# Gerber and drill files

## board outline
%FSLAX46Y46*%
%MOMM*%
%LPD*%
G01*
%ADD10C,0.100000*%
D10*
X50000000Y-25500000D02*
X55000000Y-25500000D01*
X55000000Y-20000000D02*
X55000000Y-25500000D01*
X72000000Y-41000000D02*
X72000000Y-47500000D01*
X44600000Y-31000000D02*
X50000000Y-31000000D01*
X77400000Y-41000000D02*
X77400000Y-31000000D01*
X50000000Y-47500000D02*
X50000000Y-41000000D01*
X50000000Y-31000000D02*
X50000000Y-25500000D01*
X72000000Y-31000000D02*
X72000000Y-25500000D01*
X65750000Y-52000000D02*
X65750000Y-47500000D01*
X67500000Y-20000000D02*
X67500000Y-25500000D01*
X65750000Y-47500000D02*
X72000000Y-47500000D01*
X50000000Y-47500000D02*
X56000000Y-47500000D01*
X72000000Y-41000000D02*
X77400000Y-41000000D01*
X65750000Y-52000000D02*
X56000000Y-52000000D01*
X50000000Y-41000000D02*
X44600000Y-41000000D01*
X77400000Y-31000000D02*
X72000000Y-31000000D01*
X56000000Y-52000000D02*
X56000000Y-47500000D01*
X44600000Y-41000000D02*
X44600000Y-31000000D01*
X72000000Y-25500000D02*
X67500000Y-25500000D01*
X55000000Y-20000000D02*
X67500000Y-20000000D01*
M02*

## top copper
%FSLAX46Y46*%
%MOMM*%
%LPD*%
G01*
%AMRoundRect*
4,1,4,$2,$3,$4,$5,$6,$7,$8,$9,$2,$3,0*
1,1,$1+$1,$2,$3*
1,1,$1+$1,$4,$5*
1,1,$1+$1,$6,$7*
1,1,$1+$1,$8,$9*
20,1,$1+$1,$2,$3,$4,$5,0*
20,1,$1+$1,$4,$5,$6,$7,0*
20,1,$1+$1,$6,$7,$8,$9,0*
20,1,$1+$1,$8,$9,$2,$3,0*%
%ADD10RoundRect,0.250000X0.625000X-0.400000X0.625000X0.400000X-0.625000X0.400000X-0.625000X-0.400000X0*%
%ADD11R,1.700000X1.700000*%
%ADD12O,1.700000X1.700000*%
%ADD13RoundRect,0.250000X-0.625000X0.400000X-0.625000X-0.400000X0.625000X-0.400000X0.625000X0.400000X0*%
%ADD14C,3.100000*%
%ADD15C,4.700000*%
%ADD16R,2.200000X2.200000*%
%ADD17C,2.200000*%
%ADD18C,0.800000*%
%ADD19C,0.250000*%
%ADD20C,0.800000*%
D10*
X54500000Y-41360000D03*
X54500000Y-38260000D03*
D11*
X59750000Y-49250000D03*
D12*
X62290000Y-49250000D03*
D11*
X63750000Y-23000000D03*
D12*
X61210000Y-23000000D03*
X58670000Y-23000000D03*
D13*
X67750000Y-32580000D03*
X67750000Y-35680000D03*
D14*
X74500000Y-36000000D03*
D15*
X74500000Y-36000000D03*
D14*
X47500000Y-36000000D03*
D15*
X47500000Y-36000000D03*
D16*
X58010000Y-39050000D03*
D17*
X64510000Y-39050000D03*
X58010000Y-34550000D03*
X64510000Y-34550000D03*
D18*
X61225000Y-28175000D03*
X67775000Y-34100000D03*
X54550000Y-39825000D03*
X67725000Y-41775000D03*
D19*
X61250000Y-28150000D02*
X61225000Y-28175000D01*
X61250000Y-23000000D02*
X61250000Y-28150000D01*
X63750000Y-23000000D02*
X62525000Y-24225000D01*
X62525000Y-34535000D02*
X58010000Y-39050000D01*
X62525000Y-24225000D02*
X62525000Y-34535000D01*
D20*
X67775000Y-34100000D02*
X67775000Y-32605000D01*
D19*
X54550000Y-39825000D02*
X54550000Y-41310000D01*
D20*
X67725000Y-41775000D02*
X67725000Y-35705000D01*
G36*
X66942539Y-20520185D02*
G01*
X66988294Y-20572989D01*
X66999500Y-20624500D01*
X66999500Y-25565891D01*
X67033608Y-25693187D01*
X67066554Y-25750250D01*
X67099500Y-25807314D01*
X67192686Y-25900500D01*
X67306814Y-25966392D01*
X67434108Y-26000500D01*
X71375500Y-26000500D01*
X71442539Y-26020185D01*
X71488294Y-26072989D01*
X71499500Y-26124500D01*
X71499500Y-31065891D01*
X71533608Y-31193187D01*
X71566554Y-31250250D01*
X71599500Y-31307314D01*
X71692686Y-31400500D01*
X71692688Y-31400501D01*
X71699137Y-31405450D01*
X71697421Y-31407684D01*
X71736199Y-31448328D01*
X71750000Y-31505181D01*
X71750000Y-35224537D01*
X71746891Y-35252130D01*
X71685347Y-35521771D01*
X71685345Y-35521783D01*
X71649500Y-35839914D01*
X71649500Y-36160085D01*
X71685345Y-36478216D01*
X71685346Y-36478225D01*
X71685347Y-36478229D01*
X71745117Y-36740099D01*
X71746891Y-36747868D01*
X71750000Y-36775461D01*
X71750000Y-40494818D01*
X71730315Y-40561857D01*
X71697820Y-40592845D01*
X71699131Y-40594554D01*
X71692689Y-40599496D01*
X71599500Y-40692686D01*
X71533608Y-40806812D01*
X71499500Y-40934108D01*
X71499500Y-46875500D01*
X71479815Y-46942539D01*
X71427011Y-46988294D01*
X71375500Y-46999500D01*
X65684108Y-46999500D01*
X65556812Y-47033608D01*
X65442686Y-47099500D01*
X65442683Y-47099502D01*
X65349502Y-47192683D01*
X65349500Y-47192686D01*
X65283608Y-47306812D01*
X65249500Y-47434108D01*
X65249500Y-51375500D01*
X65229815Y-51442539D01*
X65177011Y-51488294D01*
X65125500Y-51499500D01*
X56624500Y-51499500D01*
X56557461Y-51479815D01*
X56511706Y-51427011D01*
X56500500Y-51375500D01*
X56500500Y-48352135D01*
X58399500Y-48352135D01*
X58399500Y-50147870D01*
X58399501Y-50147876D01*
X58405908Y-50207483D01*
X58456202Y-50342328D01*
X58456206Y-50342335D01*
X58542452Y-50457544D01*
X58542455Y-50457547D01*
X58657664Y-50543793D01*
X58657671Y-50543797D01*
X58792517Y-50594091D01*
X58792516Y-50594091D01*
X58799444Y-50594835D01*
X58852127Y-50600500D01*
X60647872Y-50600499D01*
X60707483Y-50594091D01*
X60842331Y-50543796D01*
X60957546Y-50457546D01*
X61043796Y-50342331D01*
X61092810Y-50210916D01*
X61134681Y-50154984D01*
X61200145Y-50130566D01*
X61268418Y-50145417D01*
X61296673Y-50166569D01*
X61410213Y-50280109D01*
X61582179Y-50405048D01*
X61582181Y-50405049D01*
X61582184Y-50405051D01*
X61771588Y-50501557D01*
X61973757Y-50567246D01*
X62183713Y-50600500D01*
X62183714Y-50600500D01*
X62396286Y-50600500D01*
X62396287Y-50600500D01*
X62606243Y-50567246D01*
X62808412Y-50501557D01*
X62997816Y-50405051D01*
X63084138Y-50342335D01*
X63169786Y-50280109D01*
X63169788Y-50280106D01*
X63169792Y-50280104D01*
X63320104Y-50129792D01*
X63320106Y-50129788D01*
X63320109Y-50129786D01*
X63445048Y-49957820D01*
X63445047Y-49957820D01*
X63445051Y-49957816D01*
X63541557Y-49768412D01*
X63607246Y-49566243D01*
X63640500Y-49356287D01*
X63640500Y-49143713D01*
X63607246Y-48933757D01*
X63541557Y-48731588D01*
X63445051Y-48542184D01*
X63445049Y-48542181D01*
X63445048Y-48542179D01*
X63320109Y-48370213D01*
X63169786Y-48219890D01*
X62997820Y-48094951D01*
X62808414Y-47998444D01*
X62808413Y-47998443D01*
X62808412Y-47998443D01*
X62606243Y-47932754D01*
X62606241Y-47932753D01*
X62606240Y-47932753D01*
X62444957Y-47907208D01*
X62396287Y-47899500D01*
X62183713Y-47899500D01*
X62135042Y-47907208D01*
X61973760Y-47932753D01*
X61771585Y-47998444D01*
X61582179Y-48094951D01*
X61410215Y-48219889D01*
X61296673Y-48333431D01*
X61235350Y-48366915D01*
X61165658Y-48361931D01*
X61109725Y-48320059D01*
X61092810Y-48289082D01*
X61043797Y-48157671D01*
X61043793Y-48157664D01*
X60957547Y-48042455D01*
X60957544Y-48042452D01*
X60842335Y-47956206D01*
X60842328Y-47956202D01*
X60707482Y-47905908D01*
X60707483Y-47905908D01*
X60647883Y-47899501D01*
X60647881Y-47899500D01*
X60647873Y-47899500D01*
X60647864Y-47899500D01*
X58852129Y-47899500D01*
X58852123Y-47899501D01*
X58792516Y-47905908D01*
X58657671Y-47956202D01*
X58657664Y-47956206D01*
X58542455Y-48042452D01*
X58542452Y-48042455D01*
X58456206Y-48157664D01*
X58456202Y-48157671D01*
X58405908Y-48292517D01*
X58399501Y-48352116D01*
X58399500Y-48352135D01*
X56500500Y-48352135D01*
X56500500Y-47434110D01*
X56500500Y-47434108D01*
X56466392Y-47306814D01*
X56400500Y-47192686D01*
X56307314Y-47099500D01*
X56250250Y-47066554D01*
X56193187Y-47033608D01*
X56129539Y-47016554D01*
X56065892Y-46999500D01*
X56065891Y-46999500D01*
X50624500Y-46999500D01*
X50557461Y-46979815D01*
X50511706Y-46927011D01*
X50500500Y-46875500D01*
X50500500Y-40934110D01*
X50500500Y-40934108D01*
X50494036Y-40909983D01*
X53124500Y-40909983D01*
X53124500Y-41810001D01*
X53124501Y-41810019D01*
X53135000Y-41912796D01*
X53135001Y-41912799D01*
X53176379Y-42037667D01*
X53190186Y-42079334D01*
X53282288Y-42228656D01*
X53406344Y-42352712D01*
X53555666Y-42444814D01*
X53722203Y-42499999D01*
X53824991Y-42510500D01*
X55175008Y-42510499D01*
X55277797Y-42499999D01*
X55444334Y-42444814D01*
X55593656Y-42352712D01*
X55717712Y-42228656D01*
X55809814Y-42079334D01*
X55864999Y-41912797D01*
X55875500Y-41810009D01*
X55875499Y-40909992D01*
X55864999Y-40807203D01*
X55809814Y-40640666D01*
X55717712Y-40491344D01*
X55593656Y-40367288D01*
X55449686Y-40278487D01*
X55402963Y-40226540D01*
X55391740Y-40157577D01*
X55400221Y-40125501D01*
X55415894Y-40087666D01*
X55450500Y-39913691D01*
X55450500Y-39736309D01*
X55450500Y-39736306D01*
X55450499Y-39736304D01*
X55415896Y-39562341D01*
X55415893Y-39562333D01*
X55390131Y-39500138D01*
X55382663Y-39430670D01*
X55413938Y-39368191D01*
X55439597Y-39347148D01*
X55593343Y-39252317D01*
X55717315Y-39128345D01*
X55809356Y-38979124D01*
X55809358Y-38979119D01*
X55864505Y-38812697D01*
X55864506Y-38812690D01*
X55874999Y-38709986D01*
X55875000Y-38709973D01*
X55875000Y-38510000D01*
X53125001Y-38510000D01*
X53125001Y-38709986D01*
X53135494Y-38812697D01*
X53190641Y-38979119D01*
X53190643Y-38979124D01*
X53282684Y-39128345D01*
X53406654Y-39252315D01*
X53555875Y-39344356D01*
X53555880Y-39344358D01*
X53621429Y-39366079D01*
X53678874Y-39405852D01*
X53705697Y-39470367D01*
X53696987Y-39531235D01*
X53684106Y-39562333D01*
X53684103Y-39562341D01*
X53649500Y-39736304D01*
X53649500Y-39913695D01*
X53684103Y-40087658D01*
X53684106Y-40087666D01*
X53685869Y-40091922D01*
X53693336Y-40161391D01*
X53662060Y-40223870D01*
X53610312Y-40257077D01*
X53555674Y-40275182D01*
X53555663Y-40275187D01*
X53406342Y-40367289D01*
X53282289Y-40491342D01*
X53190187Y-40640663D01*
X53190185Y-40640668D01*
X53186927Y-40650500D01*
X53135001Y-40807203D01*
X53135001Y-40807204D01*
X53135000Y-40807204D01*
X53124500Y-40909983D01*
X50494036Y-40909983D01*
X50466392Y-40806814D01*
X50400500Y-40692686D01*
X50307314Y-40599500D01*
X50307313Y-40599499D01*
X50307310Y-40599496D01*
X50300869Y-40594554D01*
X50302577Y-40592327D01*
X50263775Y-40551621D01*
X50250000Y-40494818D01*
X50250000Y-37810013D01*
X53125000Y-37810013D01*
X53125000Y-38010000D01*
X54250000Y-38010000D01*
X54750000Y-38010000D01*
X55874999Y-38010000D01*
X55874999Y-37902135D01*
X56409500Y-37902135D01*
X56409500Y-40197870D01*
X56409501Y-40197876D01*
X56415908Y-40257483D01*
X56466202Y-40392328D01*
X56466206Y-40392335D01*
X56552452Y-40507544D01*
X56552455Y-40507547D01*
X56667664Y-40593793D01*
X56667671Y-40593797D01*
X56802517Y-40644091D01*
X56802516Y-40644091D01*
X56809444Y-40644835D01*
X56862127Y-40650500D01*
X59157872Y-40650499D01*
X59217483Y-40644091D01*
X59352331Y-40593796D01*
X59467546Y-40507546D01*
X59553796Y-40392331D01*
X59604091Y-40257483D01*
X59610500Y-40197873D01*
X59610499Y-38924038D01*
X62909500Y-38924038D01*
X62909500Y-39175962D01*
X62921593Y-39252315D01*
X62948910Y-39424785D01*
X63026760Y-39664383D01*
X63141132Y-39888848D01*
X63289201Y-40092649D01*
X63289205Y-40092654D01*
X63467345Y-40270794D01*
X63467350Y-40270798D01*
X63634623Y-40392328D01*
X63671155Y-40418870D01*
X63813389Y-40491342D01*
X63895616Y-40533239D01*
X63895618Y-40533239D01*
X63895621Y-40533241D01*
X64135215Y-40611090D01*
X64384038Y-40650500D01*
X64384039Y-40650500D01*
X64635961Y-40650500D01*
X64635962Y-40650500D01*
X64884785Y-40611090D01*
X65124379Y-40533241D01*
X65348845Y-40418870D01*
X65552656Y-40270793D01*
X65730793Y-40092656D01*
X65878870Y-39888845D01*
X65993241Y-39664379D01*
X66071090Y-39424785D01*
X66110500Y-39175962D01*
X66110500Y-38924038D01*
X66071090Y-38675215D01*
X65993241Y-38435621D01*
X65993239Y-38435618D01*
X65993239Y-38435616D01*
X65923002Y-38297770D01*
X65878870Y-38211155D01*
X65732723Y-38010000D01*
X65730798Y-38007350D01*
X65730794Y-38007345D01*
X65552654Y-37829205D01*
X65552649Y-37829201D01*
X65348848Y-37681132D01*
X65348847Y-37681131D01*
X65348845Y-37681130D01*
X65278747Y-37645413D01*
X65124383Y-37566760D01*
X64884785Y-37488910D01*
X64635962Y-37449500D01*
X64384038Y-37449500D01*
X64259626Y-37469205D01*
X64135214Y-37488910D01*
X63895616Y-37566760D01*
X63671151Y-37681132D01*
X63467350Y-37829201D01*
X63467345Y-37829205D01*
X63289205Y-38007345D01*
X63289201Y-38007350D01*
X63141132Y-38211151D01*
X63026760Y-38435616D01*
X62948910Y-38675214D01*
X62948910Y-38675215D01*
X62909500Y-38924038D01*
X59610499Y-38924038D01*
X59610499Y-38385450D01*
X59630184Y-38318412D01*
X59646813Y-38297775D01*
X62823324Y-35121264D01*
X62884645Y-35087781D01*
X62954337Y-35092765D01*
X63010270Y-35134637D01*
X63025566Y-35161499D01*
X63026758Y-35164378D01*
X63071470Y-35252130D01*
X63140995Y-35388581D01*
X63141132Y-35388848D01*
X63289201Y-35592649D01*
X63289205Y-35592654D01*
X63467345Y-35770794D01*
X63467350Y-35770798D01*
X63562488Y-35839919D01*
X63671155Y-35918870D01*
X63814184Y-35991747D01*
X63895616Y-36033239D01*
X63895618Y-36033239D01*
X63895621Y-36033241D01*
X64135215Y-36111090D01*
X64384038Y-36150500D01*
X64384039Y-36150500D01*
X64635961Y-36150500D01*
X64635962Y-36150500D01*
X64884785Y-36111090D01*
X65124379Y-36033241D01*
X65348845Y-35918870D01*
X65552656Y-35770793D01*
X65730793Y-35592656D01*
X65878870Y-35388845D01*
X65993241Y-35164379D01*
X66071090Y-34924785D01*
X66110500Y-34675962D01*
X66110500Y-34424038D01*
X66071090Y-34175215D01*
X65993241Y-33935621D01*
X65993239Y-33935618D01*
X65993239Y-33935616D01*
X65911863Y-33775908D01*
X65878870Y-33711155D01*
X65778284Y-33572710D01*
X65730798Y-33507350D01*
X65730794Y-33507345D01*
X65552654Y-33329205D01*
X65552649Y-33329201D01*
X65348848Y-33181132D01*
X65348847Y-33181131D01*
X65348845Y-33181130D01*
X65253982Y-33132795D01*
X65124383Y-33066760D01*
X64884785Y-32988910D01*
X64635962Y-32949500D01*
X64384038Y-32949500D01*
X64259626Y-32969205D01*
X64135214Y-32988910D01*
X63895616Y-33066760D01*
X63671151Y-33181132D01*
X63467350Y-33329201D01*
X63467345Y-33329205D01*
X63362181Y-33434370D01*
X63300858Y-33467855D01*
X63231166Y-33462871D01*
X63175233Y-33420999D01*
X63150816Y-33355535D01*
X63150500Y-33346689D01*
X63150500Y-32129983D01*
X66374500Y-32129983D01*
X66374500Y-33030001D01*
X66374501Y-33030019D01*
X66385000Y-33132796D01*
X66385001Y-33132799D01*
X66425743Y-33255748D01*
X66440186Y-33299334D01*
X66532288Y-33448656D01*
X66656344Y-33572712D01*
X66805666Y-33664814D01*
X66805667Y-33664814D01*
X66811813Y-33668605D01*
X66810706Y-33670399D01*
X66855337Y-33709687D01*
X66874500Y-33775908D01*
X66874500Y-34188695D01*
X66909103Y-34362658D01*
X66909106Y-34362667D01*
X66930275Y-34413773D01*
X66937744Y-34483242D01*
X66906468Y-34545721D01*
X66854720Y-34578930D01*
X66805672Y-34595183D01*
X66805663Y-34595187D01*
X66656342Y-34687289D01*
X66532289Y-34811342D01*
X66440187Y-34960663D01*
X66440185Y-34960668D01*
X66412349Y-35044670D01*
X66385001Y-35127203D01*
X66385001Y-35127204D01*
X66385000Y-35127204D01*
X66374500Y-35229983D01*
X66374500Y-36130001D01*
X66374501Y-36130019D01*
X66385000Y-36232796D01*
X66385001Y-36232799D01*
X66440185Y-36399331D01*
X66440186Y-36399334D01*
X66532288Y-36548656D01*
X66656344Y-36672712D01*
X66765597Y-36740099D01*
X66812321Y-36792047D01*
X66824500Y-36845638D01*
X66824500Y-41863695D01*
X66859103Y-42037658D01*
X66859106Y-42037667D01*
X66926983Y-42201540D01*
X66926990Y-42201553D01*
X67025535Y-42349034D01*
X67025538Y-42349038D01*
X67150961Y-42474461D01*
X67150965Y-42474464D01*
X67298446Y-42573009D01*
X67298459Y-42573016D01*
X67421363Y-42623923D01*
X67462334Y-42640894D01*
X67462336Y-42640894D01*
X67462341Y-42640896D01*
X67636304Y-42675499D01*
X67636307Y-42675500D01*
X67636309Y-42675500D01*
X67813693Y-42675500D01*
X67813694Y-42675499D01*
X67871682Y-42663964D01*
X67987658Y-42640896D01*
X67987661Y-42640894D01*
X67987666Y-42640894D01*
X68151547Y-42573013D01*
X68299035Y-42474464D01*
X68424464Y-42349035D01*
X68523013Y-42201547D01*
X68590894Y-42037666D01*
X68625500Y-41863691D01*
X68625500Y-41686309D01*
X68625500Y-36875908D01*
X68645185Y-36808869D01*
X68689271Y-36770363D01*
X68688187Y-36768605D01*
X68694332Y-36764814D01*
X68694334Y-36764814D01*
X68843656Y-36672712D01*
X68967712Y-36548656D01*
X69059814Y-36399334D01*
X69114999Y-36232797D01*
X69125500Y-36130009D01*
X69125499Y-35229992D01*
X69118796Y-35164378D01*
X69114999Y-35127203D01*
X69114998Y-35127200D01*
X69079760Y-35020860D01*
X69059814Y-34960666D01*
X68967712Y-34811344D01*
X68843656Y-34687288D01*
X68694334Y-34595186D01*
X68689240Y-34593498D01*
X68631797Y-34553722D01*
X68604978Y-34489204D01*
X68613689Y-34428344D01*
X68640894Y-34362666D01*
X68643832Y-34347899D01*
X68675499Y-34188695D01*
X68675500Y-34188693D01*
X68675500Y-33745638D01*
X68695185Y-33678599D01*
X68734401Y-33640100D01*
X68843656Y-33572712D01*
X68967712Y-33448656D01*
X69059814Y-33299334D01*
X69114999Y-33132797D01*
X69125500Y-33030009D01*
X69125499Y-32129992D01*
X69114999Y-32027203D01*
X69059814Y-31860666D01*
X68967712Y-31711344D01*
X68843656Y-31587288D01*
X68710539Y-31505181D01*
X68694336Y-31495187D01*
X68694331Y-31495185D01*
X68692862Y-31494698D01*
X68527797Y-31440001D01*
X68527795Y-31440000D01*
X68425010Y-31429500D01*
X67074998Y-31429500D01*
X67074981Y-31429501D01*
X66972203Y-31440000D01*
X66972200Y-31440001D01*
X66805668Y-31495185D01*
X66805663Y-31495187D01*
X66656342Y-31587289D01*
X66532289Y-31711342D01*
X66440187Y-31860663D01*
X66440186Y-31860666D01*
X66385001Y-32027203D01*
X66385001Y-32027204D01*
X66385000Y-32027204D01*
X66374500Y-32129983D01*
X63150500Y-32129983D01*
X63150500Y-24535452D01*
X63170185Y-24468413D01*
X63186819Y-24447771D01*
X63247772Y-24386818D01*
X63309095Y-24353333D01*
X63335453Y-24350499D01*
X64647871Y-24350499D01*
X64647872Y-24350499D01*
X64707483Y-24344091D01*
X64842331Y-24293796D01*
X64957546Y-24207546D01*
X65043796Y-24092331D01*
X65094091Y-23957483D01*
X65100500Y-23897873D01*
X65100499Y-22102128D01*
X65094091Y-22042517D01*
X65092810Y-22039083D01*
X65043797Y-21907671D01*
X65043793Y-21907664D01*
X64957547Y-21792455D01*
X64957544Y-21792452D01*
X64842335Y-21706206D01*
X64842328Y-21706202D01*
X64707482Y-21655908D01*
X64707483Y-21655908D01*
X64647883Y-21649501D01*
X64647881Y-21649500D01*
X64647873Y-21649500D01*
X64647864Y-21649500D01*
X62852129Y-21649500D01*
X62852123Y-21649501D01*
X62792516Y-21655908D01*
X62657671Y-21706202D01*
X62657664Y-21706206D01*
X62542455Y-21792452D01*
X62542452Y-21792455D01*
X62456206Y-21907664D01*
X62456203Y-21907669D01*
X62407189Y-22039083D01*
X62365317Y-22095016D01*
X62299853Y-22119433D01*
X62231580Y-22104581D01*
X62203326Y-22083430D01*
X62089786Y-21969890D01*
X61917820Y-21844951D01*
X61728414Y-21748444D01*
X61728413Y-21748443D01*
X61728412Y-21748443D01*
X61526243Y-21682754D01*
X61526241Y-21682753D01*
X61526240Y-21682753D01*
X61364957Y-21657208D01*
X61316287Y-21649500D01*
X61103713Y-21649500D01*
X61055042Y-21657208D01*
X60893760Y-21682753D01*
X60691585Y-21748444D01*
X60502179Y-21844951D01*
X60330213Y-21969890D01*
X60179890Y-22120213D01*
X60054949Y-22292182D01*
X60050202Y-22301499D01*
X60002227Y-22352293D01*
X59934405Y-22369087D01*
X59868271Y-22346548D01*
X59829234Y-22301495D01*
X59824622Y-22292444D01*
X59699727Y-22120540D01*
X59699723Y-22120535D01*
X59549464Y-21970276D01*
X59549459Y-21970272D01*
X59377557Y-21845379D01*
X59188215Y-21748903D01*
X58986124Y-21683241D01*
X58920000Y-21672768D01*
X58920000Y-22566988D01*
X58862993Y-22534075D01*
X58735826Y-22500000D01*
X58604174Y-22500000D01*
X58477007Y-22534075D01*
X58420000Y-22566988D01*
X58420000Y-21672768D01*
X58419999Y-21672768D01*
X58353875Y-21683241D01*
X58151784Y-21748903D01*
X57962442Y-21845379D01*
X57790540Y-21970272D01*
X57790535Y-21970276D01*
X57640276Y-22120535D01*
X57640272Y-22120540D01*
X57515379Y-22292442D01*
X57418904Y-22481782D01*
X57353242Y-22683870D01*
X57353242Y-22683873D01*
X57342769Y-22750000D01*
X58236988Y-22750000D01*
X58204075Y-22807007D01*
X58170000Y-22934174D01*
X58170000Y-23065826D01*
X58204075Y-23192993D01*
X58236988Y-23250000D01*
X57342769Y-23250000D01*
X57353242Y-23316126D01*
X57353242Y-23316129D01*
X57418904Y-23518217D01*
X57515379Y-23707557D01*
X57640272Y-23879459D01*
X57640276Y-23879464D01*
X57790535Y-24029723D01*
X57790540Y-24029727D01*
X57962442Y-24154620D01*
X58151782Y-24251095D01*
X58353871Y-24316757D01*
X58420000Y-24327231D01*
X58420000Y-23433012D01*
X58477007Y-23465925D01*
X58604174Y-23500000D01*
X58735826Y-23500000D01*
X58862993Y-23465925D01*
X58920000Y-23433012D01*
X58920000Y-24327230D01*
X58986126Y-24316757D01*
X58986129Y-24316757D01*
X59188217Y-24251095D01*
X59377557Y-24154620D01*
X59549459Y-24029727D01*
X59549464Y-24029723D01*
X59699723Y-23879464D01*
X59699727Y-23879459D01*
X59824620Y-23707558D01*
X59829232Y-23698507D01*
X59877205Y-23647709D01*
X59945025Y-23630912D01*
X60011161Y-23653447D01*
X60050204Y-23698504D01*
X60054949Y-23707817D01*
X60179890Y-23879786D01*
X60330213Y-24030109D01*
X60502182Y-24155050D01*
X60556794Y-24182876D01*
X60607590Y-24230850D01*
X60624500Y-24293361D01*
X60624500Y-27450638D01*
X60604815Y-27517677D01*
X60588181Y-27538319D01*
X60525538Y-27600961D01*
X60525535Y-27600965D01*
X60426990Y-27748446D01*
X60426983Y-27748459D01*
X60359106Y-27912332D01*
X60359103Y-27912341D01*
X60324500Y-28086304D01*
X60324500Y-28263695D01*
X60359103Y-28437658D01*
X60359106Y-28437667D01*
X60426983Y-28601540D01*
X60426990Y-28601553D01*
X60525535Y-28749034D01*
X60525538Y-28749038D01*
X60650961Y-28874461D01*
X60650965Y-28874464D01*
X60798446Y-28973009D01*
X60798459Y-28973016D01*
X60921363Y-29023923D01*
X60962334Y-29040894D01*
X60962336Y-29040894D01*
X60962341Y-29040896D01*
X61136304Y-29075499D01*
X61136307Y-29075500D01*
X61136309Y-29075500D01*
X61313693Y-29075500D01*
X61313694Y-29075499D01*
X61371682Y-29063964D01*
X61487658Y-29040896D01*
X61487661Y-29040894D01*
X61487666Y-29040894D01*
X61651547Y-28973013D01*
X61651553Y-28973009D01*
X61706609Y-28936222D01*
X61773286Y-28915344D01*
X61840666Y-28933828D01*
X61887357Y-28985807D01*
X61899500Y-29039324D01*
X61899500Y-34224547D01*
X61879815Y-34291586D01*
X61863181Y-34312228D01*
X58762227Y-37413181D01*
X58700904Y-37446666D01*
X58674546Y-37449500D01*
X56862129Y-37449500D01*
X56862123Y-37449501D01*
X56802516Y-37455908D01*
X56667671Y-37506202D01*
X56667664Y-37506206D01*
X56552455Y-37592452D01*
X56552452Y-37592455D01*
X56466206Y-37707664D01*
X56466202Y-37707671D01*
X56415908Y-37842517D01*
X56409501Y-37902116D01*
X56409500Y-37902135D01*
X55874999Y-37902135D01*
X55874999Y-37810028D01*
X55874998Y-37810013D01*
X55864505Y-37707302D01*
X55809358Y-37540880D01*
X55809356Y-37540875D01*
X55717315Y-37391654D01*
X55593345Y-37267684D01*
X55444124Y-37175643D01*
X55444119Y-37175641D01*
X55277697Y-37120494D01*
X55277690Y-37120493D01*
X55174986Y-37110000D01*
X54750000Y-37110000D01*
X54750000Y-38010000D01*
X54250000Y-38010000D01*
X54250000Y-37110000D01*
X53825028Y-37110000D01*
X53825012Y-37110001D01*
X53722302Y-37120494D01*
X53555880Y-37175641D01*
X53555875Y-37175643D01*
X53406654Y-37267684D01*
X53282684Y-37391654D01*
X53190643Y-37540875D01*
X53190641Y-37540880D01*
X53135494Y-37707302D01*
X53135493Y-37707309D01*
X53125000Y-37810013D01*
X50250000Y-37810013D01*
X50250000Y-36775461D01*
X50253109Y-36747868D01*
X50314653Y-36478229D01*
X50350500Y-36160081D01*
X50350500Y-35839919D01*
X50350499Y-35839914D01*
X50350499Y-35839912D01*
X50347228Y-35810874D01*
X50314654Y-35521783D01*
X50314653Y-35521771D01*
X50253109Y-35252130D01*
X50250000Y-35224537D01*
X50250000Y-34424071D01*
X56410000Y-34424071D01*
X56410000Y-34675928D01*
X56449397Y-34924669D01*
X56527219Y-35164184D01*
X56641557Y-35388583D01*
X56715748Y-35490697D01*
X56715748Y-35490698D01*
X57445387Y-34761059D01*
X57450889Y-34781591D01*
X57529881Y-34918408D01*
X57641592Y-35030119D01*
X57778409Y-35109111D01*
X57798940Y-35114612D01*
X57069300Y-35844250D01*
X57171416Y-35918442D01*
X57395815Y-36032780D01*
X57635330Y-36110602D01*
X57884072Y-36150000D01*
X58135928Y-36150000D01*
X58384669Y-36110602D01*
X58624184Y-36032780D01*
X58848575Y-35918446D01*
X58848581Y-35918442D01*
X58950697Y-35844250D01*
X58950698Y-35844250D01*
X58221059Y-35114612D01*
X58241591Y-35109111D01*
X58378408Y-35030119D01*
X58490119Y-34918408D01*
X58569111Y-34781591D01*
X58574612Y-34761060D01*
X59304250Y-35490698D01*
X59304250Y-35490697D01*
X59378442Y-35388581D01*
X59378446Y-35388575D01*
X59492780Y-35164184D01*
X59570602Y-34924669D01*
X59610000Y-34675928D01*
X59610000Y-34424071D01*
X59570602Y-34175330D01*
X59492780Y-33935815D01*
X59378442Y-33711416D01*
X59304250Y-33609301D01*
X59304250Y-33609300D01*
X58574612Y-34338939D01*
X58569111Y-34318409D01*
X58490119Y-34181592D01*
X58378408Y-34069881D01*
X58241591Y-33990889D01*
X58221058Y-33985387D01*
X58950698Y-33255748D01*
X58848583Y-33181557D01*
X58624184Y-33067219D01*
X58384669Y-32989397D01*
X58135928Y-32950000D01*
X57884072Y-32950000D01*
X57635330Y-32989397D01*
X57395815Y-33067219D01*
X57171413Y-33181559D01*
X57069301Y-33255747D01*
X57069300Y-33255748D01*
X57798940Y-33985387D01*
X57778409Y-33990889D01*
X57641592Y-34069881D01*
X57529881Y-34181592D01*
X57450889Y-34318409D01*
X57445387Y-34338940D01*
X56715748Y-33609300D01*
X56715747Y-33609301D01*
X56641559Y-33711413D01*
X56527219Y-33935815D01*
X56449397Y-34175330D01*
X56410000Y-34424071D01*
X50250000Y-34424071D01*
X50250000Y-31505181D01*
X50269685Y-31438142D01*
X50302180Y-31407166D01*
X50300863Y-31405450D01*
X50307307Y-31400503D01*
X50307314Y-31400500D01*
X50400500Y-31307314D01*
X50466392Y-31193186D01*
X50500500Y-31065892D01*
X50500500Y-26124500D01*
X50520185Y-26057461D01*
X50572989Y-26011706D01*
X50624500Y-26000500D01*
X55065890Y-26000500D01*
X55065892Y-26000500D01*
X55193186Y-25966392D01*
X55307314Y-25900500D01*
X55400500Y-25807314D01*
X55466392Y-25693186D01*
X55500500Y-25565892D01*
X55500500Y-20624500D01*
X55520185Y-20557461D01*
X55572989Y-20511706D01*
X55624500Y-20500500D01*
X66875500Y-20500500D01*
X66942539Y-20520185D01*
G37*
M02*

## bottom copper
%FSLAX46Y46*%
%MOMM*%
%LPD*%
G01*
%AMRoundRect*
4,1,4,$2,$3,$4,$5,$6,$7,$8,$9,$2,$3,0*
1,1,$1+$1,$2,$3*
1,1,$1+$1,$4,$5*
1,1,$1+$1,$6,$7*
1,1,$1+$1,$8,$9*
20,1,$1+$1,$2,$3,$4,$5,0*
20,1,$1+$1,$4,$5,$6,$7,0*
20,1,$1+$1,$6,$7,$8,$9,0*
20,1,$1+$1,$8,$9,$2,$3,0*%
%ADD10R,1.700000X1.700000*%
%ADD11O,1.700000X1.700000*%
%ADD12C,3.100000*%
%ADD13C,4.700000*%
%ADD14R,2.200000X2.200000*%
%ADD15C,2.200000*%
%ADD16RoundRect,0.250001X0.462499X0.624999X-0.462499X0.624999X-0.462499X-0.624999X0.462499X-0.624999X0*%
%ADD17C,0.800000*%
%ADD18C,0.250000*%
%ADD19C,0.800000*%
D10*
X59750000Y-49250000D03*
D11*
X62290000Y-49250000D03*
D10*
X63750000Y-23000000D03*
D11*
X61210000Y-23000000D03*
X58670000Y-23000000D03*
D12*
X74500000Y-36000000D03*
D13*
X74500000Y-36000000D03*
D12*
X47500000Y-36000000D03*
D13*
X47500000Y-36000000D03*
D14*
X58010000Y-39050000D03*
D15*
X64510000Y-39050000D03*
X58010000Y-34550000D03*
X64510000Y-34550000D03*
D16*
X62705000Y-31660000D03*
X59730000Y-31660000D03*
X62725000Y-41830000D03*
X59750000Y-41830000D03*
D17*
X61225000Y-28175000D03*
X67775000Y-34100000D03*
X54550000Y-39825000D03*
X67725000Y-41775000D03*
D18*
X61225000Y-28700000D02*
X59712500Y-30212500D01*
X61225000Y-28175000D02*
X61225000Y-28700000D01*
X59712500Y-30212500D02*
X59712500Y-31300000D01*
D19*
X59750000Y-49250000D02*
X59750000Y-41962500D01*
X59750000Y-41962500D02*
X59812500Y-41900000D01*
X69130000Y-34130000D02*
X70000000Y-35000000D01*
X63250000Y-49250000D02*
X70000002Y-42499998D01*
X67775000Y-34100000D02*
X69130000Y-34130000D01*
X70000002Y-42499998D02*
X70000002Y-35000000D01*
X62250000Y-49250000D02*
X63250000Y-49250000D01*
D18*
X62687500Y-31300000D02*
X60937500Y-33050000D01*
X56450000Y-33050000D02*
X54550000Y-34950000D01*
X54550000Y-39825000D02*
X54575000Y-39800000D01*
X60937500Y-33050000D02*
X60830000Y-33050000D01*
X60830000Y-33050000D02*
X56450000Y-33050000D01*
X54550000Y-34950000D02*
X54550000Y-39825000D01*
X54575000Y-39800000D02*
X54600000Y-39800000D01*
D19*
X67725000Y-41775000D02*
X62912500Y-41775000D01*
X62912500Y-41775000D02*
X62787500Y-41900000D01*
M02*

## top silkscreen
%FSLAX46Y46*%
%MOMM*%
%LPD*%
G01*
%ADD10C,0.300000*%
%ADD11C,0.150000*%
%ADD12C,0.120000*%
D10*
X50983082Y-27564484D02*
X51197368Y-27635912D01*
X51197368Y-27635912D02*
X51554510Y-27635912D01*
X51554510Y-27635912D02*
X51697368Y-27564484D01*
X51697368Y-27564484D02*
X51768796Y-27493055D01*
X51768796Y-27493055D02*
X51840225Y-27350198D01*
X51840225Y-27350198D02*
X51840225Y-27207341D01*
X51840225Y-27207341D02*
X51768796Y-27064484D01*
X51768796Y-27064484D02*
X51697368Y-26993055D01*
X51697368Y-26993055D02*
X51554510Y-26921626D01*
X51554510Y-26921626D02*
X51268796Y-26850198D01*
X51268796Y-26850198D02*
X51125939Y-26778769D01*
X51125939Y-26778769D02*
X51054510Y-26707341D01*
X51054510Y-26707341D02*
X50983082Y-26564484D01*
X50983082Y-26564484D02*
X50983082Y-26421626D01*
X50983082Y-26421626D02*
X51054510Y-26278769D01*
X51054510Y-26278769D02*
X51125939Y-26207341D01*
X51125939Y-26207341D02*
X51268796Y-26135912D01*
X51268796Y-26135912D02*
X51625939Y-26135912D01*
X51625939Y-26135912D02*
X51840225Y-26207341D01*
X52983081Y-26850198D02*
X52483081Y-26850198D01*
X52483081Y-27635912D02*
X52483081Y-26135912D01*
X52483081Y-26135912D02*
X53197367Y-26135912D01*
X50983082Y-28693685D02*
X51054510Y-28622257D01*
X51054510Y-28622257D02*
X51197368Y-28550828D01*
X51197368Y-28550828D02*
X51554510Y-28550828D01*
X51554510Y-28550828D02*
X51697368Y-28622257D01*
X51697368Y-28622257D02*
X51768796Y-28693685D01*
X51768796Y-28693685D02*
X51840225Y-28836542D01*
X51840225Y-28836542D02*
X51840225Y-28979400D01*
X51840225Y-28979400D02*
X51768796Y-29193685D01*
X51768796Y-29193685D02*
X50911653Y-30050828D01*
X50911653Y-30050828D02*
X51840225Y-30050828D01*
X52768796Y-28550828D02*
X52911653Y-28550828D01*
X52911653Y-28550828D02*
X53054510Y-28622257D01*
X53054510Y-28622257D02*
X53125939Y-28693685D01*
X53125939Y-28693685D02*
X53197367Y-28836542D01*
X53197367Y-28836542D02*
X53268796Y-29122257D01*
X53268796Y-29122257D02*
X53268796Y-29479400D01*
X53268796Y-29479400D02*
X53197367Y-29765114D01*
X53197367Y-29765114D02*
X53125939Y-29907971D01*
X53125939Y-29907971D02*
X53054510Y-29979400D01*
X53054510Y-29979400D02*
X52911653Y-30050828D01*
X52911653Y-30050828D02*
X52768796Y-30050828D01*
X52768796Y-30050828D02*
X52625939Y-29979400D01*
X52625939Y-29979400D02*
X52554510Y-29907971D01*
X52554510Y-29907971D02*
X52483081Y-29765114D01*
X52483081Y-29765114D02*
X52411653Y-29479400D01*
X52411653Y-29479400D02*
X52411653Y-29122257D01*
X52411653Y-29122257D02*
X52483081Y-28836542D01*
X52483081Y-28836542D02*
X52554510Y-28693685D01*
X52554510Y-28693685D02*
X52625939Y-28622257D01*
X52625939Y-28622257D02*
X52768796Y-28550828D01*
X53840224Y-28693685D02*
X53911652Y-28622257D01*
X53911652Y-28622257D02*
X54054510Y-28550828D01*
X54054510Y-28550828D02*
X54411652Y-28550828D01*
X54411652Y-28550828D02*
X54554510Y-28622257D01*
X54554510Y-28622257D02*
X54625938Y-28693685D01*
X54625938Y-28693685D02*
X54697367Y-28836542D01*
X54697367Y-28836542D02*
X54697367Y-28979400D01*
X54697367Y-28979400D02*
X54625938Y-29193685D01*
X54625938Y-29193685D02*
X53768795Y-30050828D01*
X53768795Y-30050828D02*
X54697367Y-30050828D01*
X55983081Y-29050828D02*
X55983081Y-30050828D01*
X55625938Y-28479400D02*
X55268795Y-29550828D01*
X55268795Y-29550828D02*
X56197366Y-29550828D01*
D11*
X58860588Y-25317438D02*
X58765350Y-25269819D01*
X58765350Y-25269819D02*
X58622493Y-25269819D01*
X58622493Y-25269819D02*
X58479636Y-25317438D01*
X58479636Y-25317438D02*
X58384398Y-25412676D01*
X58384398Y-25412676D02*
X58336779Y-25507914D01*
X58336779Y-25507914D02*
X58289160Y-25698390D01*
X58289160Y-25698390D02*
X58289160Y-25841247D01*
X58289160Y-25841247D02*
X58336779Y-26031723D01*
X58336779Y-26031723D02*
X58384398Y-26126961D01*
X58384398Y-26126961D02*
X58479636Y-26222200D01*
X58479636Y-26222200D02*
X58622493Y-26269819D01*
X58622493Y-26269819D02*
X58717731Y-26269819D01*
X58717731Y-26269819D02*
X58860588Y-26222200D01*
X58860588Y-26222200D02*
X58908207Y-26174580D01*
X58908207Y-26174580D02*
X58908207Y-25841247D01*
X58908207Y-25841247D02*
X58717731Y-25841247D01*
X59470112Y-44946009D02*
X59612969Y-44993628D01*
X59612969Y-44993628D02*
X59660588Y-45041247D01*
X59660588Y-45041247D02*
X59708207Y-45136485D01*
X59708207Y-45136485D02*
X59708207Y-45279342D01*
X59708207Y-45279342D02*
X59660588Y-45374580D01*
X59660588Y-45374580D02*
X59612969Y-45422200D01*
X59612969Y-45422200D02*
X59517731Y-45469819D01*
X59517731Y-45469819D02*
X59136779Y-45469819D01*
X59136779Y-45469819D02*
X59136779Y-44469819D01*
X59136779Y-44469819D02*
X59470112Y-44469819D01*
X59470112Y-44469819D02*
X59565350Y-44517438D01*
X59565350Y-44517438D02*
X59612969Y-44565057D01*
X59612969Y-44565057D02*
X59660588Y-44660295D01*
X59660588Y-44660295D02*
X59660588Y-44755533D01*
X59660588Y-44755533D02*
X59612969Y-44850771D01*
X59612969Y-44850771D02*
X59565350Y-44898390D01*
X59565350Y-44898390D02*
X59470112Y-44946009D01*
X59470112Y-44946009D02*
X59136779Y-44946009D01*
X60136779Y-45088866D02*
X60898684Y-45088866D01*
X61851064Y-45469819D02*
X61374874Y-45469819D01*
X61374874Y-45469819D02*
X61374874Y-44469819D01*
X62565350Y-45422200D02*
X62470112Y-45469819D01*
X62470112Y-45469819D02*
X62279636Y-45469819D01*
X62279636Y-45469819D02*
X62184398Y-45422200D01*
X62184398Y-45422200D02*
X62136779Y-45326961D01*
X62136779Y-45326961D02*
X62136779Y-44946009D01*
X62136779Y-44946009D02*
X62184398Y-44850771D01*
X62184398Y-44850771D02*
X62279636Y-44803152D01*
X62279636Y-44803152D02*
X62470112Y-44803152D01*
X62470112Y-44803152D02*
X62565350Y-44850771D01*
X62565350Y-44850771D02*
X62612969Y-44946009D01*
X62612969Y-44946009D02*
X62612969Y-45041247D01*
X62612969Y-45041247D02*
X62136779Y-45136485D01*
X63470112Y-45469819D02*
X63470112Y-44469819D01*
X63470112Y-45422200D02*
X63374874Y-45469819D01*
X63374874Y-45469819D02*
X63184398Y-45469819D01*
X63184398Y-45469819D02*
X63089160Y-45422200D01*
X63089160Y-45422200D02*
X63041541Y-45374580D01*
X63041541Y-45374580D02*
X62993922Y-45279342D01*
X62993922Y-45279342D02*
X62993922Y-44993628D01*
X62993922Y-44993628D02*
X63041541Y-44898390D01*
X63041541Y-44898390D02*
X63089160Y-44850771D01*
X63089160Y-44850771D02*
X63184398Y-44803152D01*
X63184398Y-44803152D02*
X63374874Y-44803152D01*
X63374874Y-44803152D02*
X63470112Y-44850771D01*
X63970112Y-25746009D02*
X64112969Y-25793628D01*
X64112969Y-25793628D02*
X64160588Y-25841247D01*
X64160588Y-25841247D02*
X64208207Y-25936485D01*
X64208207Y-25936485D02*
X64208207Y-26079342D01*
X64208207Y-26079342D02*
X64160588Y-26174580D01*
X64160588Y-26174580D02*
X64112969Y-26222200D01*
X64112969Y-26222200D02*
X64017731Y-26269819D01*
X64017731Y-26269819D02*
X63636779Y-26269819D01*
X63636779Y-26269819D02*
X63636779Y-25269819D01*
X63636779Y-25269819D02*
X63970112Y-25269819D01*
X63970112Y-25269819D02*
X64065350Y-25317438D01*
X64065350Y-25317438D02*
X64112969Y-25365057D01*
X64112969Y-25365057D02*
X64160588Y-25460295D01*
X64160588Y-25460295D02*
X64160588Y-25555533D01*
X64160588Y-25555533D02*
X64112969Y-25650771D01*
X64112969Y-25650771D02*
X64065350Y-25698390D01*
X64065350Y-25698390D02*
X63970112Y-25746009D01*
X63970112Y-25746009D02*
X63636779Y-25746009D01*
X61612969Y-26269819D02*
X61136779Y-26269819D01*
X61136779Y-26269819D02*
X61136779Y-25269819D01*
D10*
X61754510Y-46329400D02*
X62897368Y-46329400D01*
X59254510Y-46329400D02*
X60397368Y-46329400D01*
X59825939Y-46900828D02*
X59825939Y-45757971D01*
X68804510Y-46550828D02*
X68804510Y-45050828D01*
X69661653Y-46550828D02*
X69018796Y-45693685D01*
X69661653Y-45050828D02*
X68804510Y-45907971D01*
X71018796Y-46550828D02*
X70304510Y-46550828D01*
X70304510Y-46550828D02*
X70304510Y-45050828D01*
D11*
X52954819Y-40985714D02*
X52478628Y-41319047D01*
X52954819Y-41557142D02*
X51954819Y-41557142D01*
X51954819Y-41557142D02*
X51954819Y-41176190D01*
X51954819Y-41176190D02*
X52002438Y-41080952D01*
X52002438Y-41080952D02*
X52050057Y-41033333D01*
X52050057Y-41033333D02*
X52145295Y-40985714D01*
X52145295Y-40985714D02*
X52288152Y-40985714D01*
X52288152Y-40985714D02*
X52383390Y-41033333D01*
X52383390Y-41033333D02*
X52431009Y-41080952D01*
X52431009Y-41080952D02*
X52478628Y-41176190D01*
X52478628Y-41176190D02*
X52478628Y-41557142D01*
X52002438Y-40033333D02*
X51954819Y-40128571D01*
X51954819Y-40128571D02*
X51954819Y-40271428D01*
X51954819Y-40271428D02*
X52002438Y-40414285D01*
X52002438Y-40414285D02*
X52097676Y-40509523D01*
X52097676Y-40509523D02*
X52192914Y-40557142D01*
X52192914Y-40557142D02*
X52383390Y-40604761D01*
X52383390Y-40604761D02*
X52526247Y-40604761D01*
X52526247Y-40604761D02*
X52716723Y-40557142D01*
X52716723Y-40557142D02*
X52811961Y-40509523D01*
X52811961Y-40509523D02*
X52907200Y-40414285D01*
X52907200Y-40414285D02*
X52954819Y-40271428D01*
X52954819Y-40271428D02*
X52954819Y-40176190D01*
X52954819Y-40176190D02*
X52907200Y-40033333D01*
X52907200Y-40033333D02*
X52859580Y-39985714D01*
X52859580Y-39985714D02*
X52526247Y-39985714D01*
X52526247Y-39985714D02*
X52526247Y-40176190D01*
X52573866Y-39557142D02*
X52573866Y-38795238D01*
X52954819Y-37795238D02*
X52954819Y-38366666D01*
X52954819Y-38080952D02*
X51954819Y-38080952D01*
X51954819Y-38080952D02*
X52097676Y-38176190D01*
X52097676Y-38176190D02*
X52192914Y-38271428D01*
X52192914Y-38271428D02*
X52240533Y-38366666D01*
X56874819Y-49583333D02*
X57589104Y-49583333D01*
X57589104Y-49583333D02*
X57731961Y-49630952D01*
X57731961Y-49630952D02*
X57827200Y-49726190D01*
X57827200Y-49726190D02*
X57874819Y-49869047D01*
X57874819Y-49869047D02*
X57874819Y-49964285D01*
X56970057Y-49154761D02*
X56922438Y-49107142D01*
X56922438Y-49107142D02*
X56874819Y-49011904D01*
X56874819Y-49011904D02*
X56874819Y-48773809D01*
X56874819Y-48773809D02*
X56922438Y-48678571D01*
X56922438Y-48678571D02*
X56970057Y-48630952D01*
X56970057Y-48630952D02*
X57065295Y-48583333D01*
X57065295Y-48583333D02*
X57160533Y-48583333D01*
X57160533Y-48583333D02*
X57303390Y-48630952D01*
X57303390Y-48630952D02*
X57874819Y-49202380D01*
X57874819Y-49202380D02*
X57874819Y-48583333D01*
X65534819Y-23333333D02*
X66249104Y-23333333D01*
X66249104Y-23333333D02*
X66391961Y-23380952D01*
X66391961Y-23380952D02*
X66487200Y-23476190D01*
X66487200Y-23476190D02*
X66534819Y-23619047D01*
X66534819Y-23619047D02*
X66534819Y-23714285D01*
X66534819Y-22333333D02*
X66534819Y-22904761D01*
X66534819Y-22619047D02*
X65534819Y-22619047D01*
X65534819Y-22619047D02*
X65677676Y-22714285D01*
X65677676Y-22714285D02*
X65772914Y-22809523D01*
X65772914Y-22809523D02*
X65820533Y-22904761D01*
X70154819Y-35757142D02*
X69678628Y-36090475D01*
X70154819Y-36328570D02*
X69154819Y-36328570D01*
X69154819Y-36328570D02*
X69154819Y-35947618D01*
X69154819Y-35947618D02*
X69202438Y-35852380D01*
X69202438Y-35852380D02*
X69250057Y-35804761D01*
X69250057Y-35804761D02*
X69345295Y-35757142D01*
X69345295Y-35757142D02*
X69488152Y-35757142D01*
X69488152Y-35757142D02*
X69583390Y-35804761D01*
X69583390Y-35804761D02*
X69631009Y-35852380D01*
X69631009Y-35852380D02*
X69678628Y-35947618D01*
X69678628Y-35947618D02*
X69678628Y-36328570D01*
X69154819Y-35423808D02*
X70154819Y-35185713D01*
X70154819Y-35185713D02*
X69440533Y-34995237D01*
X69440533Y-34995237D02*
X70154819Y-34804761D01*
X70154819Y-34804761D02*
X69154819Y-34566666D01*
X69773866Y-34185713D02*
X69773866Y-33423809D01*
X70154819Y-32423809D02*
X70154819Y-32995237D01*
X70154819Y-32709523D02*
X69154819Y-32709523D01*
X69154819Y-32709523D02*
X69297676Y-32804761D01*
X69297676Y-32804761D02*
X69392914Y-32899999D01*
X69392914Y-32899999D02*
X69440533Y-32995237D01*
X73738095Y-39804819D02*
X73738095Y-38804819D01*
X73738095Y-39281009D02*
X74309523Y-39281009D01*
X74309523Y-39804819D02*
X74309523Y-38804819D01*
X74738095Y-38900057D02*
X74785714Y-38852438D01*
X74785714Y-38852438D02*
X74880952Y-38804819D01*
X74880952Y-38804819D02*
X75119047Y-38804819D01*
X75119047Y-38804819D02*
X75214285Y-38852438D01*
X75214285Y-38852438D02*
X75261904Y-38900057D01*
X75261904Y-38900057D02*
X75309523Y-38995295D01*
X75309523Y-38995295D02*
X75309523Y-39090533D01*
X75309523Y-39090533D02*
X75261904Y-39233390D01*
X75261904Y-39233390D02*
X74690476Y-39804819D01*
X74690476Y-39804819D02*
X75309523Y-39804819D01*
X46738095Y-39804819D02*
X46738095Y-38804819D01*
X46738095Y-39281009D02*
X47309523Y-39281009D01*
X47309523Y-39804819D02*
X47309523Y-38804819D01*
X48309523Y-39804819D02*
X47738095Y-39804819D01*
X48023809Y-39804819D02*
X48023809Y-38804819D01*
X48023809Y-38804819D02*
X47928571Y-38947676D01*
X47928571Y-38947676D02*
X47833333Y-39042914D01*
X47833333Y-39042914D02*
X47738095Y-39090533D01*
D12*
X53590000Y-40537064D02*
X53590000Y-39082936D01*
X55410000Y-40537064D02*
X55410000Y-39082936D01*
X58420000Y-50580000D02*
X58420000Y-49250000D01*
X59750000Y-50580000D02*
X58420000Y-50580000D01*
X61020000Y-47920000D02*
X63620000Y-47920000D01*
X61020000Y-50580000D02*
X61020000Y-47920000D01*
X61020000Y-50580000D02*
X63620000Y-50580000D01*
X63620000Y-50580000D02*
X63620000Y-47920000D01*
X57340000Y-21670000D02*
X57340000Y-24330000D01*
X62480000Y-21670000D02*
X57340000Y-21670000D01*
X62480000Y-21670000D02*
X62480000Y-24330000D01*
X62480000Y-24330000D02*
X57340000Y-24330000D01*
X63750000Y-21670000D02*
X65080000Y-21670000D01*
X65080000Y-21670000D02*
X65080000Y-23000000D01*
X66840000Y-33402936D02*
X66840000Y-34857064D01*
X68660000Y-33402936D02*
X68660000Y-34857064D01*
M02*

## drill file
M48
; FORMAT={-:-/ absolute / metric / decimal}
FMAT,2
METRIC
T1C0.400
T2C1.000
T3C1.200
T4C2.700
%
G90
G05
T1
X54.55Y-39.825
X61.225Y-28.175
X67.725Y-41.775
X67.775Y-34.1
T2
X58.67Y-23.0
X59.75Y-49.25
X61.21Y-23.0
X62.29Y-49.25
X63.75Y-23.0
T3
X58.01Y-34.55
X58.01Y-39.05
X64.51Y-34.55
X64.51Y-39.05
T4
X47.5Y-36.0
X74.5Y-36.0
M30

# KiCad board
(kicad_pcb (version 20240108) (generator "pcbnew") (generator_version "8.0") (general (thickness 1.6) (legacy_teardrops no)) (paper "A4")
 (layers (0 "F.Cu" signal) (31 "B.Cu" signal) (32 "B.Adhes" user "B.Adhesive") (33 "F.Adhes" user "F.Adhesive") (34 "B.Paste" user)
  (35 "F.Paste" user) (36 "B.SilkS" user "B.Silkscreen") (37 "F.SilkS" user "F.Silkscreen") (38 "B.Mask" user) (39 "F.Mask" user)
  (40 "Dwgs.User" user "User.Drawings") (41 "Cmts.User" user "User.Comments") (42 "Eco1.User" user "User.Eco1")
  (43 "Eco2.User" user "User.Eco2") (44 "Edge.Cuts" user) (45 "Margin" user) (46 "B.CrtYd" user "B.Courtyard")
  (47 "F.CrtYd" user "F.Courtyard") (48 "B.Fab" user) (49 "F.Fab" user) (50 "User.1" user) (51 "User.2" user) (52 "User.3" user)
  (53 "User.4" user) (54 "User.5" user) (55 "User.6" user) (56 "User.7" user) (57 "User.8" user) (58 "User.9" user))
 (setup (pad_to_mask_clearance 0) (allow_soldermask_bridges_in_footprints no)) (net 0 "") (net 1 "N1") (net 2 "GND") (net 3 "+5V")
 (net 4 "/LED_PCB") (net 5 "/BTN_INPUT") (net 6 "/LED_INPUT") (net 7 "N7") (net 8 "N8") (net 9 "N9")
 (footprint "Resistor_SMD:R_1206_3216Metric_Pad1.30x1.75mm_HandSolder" (layer "F.Cu") (at 54.5 39.81 90)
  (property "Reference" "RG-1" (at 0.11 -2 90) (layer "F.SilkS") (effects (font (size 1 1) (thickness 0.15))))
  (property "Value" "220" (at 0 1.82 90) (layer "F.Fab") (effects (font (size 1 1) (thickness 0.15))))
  (fp_line (start -0.727064 -0.91) (end 0.727064 -0.91) (stroke (width 0.12) (type solid)) (layer "F.SilkS"))
  (fp_line (start -0.727064 0.91) (end 0.727064 0.91) (stroke (width 0.12) (type solid)) (layer "F.SilkS"))
  (pad "1" smd roundrect (at -1.55 0 90) (size 1.3 1.75) (layers "F.Cu" "F.Paste" "F.Mask") (roundrect_rratio 0.192308) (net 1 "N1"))
  (pad "2" smd roundrect (at 1.55 0 90) (size 1.3 1.75) (layers "F.Cu" "F.Paste" "F.Mask") (roundrect_rratio 0.192308) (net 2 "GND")))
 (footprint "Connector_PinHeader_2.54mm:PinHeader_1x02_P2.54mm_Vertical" (layer "F.Cu") (at 59.75 49.25 90)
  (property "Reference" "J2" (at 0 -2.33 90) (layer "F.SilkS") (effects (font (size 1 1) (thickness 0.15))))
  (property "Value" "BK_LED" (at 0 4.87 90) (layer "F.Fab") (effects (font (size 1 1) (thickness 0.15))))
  (fp_line (start -1.33 -1.33) (end 0 -1.33) (stroke (width 0.12) (type solid)) (layer "F.SilkS"))
  (fp_line (start -1.33 0) (end -1.33 -1.33) (stroke (width 0.12) (type solid)) (layer "F.SilkS"))
  (fp_line (start 1.33 1.27) (end 1.33 3.87) (stroke (width 0.12) (type solid)) (layer "F.SilkS"))
  (fp_line (start -1.33 1.27) (end 1.33 1.27) (stroke (width 0.12) (type solid)) (layer "F.SilkS"))
  (fp_line (start -1.33 1.27) (end -1.33 3.87) (stroke (width 0.12) (type solid)) (layer "F.SilkS"))
  (fp_line (start -1.33 3.87) (end 1.33 3.87) (stroke (width 0.12) (type solid)) (layer "F.SilkS"))
  (pad "1" thru_hole rect (at 0 0 90) (size 1.7 1.7) (drill 1) (layers "*.Cu" "*.Mask") (remove_unused_layers no) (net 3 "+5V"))
  (pad "2" thru_hole oval (at 0 2.54 90) (size 1.7 1.7) (drill 1) (layers "*.Cu" "*.Mask") (remove_unused_layers no) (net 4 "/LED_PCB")))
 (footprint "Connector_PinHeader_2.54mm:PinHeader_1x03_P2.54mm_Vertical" (layer "F.Cu") (at 63.75 23 -90)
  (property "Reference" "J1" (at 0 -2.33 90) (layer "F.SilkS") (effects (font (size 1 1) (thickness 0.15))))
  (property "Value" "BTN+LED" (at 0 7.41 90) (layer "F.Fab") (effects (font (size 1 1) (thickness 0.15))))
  (fp_line (start -1.33 6.41) (end 1.33 6.41) (stroke (width 0.12) (type solid)) (layer "F.SilkS"))
  (fp_line (start -1.33 1.27) (end -1.33 6.41) (stroke (width 0.12) (type solid)) (layer "F.SilkS"))
  (fp_line (start -1.33 1.27) (end 1.33 1.27) (stroke (width 0.12) (type solid)) (layer "F.SilkS"))
  (fp_line (start 1.33 1.27) (end 1.33 6.41) (stroke (width 0.12) (type solid)) (layer "F.SilkS"))
  (fp_line (start -1.33 0) (end -1.33 -1.33) (stroke (width 0.12) (type solid)) (layer "F.SilkS"))
  (fp_line (start -1.33 -1.33) (end 0 -1.33) (stroke (width 0.12) (type solid)) (layer "F.SilkS"))
  (pad "1" thru_hole rect (at 0 0 270) (size 1.7 1.7) (drill 1) (layers "*.Cu" "*.Mask") (remove_unused_layers no) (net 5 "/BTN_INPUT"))
  (pad "2" thru_hole oval (at 0 2.54 270) (size 1.7 1.7) (drill 1) (layers "*.Cu" "*.Mask") (remove_unused_layers no) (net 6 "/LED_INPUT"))
  (pad "3" thru_hole oval (at 0 5.08 270) (size 1.7 1.7) (drill 1) (layers "*.Cu" "*.Mask") (remove_unused_layers no) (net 2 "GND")))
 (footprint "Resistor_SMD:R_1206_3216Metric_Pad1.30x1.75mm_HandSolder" (layer "F.Cu") (at 67.75 34.13 -90)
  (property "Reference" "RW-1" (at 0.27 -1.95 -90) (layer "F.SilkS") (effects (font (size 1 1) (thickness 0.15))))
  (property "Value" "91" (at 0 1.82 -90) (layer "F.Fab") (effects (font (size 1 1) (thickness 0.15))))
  (fp_line (start -0.727064 0.91) (end 0.727064 0.91) (stroke (width 0.12) (type solid)) (layer "F.SilkS"))
  (fp_line (start -0.727064 -0.91) (end 0.727064 -0.91) (stroke (width 0.12) (type solid)) (layer "F.SilkS"))
  (pad "1" smd roundrect (at -1.55 0 270) (size 1.3 1.75) (layers "F.Cu" "F.Paste" "F.Mask") (roundrect_rratio 0.192308) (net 4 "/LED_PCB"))
  (pad "2" smd roundrect (at 1.55 0 270) (size 1.3 1.75) (layers "F.Cu" "F.Paste" "F.Mask") (roundrect_rratio 0.192308) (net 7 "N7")))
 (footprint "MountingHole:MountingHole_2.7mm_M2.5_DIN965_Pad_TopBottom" (layer "F.Cu") (at 74.5 36 180)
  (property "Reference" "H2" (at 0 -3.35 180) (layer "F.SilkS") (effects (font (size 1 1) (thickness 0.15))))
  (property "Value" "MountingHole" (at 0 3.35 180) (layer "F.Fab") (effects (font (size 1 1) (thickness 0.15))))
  (pad "1" thru_hole circle (at 0 0 180) (size 3.1 3.1) (drill 2.7) (layers "*.Cu" "*.Mask") (remove_unused_layers no))
  (pad "1" connect circle (at 0 0 180) (size 4.7 4.7) (layers "F.Cu" "F.Mask"))
  (pad "1" connect circle (at 0 0 180) (size 4.7 4.7) (layers "B.Cu" "B.Mask")))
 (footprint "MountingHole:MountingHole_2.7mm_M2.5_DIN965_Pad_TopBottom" (layer "F.Cu") (at 47.5 36 180)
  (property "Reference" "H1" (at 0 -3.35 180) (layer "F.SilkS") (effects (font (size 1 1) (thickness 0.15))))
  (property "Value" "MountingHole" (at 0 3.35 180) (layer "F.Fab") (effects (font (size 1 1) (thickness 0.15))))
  (pad "1" thru_hole circle (at 0 0 180) (size 3.1 3.1) (drill 2.7) (layers "*.Cu" "*.Mask") (remove_unused_layers no))
  (pad "1" connect circle (at 0 0 180) (size 4.7 4.7) (layers "F.Cu" "F.Mask"))
  (pad "1" connect circle (at 0 0 180) (size 4.7 4.7) (layers "B.Cu" "B.Mask")))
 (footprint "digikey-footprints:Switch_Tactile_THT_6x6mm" (layer "B.Cu") (at 58.01 39.05)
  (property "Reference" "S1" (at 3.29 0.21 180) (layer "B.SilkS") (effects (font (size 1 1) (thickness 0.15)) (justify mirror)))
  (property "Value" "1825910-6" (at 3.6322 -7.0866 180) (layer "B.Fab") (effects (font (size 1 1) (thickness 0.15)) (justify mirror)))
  (pad "1" thru_hole rect (at 0 0) (size 2.2 2.2) (drill 1.2) (layers "*.Cu" "*.Mask") (remove_unused_layers no) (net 5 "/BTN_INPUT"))
  (pad "2" thru_hole circle (at 6.5 0) (size 2.2 2.2) (drill 1.2) (layers "*.Cu" "*.Mask") (remove_unused_layers no) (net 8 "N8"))
  (pad "3" thru_hole circle (at 0 -4.5) (size 2.2 2.2) (drill 1.2) (layers "*.Cu" "*.Mask") (remove_unused_layers no) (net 2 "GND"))
  (pad "4" thru_hole circle (at 6.5 -4.5) (size 2.2 2.2) (drill 1.2) (layers "*.Cu" "*.Mask") (remove_unused_layers no) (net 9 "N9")))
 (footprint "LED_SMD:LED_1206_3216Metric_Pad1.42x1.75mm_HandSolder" (layer "B.Cu") (at 61.2175 31.66 180)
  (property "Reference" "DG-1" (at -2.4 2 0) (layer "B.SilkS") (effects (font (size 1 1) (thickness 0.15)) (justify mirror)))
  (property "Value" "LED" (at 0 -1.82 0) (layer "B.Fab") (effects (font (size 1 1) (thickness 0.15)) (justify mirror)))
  (pad "1" smd roundrect (at -1.4875 0 180) (size 1.425 1.75) (layers "B.Cu" "B.Paste" "B.Mask") (roundrect_rratio 0.175439) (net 1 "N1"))
  (pad "2" smd roundrect (at 1.4875 0 180) (size 1.425 1.75) (layers "B.Cu" "B.Paste" "B.Mask") (roundrect_rratio 0.175439)
   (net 6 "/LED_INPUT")))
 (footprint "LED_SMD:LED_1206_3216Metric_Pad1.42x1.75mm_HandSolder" (layer "B.Cu") (at 61.2375 41.83 180)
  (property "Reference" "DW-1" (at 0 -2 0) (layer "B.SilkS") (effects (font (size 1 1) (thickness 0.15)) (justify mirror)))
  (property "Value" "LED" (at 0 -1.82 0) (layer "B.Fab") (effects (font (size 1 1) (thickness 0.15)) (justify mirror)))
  (pad "1" smd roundrect (at -1.4875 0 180) (size 1.425 1.75) (layers "B.Cu" "B.Paste" "B.Mask") (roundrect_rratio 0.175439) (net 7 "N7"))
  (pad "2" smd roundrect (at 1.4875 0 180) (size 1.425 1.75) (layers "B.Cu" "B.Paste" "B.Mask") (roundrect_rratio 0.175439) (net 3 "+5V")))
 (gr_line (start 50 25.5) (end 55 25.5) (stroke (width 0.1) (type default)) (layer "Edge.Cuts"))
 (gr_line (start 55 20) (end 55 25.5) (stroke (width 0.1) (type default)) (layer "Edge.Cuts"))
 (gr_line (start 72 41) (end 72 47.5) (stroke (width 0.1) (type default)) (layer "Edge.Cuts"))
 (gr_line (start 44.6 31) (end 50 31) (stroke (width 0.1) (type default)) (layer "Edge.Cuts"))
 (gr_line (start 77.4 41) (end 77.4 31) (stroke (width 0.1) (type default)) (layer "Edge.Cuts"))
 (gr_line (start 50 47.5) (end 50 41) (stroke (width 0.1) (type default)) (layer "Edge.Cuts"))
 (gr_line (start 50 31) (end 50 25.5) (stroke (width 0.1) (type default)) (layer "Edge.Cuts"))
 (gr_line (start 72 31) (end 72 25.5) (stroke (width 0.1) (type default)) (layer "Edge.Cuts"))
 (gr_line (start 65.75 52) (end 65.75 47.5) (stroke (width 0.1) (type default)) (layer "Edge.Cuts"))
 (gr_line (start 67.5 20) (end 67.5 25.5) (stroke (width 0.1) (type default)) (layer "Edge.Cuts"))
 (gr_line (start 65.75 47.5) (end 72 47.5) (stroke (width 0.1) (type default)) (layer "Edge.Cuts"))
 (gr_line (start 50 47.5) (end 56 47.5) (stroke (width 0.1) (type default)) (layer "Edge.Cuts"))
 (gr_line (start 72 41) (end 77.4 41) (stroke (width 0.1) (type default)) (layer "Edge.Cuts"))
 (gr_line (start 65.75 52) (end 56 52) (stroke (width 0.1) (type default)) (layer "Edge.Cuts"))
 (gr_line (start 50 41) (end 44.6 41) (stroke (width 0.1) (type default)) (layer "Edge.Cuts"))
 (gr_line (start 77.4 31) (end 72 31) (stroke (width 0.1) (type default)) (layer "Edge.Cuts"))
 (gr_line (start 56 52) (end 56 47.5) (stroke (width 0.1) (type default)) (layer "Edge.Cuts"))
 (gr_line (start 44.6 41) (end 44.6 31) (stroke (width 0.1) (type default)) (layer "Edge.Cuts"))
 (gr_line (start 72 25.5) (end 67.5 25.5) (stroke (width 0.1) (type default)) (layer "Edge.Cuts"))
 (gr_line (start 55 20) (end 67.5 20) (stroke (width 0.1) (type default)) (layer "Edge.Cuts"))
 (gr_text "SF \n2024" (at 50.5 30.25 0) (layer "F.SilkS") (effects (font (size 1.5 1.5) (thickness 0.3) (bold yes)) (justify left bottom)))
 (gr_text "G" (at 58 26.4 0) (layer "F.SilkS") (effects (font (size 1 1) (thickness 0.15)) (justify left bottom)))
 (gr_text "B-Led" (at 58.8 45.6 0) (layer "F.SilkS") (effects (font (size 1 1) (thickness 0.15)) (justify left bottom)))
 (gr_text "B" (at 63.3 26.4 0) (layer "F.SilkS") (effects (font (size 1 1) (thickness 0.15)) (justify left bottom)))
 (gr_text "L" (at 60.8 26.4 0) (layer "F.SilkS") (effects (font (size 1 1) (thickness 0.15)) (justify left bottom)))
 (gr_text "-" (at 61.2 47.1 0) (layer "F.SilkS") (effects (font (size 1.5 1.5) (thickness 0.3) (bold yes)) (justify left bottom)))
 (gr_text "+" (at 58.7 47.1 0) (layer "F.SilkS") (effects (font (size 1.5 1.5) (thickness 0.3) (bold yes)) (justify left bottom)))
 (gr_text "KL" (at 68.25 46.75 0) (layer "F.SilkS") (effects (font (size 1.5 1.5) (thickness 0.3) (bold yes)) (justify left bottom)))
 (segment (start 61.25 28.15) (end 61.225 28.175) (width 0.25) (layer "F.Cu") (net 6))
 (segment (start 61.25 23) (end 61.25 28.15) (width 0.25) (layer "F.Cu") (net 6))
 (via (at 61.225 28.175) (size 0.8) (drill 0.4) (layers "F.Cu" "B.Cu") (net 6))
 (segment (start 61.225 28.7) (end 59.7125 30.2125) (width 0.25) (layer "B.Cu") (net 6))
 (segment (start 61.225 28.175) (end 61.225 28.7) (width 0.25) (layer "B.Cu") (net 6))
 (segment (start 59.7125 30.2125) (end 59.7125 31.3) (width 0.25) (layer "B.Cu") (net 6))
 (segment (start 59.75 49.25) (end 59.75 41.9625) (width 0.8) (layer "B.Cu") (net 3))
 (segment (start 59.75 41.9625) (end 59.8125 41.9) (width 0.8) (layer "B.Cu") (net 3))
 (segment (start 63.75 23) (end 62.525 24.225) (width 0.25) (layer "F.Cu") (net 5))
 (segment (start 62.525 34.535) (end 58.01 39.05) (width 0.25) (layer "F.Cu") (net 5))
 (segment (start 62.525 24.225) (end 62.525 34.535) (width 0.25) (layer "F.Cu") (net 5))
 (segment (start 67.775 34.1) (end 67.775 32.605) (width 0.8) (layer "F.Cu") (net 4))
 (via (at 67.775 34.1) (size 0.8) (drill 0.4) (layers "F.Cu" "B.Cu") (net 4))
 (segment (start 69.13 34.13) (end 70 35) (width 0.8) (layer "B.Cu") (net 4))
 (segment (start 63.25 49.25) (end 70.000002 42.499998) (width 0.8) (layer "B.Cu") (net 4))
 (segment (start 67.775 34.1) (end 69.13 34.13) (width 0.8) (layer "B.Cu") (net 4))
 (segment (start 70.000002 42.499998) (end 70.000002 35) (width 0.8) (layer "B.Cu") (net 4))
 (segment (start 62.25 49.25) (end 63.25 49.25) (width 0.8) (layer "B.Cu") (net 4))
 (segment (start 54.55 39.825) (end 54.55 41.31) (width 0.25) (layer "F.Cu") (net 1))
 (via (at 54.55 39.825) (size 0.8) (drill 0.4) (layers "F.Cu" "B.Cu") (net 1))
 (segment (start 62.6875 31.3) (end 60.9375 33.05) (width 0.25) (layer "B.Cu") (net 1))
 (segment (start 56.45 33.05) (end 54.55 34.95) (width 0.25) (layer "B.Cu") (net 1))
 (segment (start 54.55 39.825) (end 54.575 39.8) (width 0.25) (layer "B.Cu") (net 1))
 (segment (start 60.9375 33.05) (end 60.83 33.05) (width 0.25) (layer "B.Cu") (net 1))
 (segment (start 60.83 33.05) (end 56.45 33.05) (width 0.25) (layer "B.Cu") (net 1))
 (segment (start 54.55 34.95) (end 54.55 39.825) (width 0.25) (layer "B.Cu") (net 1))
 (segment (start 54.575 39.8) (end 54.6 39.8) (width 0.25) (layer "B.Cu") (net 1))
 (segment (start 67.725 41.775) (end 67.725 35.705) (width 0.8) (layer "F.Cu") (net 7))
 (via (at 67.725 41.775) (size 0.8) (drill 0.4) (layers "F.Cu" "B.Cu") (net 7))
 (segment (start 67.725 41.775) (end 62.9125 41.775) (width 0.8) (layer "B.Cu") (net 7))
 (segment (start 62.9125 41.775) (end 62.7875 41.9) (width 0.8) (layer "B.Cu") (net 7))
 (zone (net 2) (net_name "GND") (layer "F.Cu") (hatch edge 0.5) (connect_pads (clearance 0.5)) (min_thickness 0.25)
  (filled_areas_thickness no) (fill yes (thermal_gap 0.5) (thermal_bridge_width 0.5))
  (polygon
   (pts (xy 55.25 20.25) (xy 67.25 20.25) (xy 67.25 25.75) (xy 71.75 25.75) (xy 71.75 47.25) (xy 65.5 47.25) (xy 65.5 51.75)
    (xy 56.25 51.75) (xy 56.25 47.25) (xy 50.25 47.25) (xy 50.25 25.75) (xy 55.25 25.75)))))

